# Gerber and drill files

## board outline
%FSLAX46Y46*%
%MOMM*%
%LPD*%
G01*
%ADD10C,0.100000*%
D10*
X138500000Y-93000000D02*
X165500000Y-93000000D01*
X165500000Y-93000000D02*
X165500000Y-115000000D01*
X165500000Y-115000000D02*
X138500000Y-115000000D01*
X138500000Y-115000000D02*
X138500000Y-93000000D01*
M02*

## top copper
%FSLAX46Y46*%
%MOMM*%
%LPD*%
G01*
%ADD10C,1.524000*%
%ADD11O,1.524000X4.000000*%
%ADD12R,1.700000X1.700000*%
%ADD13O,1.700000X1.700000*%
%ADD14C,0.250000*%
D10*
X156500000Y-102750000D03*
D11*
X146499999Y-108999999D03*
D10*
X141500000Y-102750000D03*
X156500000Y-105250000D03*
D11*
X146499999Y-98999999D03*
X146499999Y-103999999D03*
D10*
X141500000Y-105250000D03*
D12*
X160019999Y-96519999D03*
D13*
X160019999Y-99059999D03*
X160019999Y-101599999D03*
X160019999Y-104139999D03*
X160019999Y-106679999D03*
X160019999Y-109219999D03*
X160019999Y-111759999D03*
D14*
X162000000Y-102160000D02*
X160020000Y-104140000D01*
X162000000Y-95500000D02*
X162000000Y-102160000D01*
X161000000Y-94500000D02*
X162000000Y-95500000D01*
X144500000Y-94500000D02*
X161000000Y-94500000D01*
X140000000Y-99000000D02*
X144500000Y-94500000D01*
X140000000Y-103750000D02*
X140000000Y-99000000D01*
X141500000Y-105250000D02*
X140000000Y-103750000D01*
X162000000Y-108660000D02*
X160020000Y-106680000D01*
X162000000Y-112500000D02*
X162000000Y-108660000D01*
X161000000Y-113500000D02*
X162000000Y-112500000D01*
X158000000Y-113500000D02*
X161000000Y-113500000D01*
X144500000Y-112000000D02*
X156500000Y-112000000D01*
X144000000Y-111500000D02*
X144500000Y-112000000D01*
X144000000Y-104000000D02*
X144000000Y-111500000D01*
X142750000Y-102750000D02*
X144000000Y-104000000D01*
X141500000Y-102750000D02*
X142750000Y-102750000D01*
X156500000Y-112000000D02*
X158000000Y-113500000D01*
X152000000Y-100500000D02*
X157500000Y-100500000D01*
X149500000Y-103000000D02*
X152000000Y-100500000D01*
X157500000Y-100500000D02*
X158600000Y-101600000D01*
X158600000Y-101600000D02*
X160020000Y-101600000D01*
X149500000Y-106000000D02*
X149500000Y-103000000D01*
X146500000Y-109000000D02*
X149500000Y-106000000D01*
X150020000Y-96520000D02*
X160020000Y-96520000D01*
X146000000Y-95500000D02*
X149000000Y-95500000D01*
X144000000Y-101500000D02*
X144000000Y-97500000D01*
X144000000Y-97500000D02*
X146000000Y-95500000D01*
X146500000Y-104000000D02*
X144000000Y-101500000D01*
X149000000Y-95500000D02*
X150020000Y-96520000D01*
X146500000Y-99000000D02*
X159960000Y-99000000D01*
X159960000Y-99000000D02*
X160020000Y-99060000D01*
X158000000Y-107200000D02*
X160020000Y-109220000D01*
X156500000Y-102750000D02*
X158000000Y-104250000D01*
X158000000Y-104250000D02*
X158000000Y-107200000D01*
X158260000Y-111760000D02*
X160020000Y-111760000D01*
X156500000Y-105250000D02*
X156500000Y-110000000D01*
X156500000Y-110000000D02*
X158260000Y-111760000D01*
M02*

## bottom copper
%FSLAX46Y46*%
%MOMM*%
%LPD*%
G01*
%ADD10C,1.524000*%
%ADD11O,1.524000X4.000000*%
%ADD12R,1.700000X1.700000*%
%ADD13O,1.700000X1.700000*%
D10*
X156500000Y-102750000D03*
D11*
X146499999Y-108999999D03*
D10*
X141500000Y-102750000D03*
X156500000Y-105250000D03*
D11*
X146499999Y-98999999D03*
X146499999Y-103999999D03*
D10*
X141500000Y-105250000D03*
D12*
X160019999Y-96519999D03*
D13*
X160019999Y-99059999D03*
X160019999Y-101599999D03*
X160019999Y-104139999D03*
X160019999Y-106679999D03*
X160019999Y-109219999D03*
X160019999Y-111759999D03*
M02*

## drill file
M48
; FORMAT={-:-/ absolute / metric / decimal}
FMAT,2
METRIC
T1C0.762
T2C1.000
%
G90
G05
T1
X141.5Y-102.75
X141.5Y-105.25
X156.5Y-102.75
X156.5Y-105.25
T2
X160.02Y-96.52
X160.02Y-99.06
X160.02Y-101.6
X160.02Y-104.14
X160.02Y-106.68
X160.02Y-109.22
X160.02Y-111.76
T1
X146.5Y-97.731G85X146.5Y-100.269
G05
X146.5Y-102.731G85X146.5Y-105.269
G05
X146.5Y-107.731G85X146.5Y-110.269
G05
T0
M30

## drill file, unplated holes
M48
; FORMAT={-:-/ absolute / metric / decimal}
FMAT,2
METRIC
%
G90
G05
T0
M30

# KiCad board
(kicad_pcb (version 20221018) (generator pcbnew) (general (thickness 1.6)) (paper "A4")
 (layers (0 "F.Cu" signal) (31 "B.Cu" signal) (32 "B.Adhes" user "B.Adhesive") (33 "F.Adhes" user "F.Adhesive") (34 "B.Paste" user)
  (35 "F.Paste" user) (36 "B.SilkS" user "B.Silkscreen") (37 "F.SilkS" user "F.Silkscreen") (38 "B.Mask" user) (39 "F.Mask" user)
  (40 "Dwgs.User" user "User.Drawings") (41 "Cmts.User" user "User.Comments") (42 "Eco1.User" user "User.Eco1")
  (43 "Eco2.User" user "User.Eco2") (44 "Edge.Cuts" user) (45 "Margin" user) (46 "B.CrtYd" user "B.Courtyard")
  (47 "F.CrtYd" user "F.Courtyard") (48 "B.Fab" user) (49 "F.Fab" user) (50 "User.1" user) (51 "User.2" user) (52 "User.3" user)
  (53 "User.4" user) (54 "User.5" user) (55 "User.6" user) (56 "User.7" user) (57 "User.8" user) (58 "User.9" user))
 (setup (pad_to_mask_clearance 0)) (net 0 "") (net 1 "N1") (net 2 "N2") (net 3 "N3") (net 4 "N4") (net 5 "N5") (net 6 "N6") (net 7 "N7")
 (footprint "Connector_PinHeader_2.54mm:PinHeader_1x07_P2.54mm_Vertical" (layer "F.Cu") (at 160.02 96.52)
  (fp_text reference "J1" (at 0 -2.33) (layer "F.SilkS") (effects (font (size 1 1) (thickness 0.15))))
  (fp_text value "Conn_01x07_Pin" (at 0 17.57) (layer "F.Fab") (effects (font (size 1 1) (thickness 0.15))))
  (pad "1" thru_hole rect (at 0 0) (size 1.7 1.7) (drill 1) (layers "*.Cu" "*.Mask") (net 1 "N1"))
  (pad "2" thru_hole oval (at 0 2.54) (size 1.7 1.7) (drill 1) (layers "*.Cu" "*.Mask") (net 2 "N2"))
  (pad "3" thru_hole oval (at 0 5.08) (size 1.7 1.7) (drill 1) (layers "*.Cu" "*.Mask") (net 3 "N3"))
  (pad "4" thru_hole oval (at 0 7.62) (size 1.7 1.7) (drill 1) (layers "*.Cu" "*.Mask") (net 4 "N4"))
  (pad "5" thru_hole oval (at 0 10.16) (size 1.7 1.7) (drill 1) (layers "*.Cu" "*.Mask") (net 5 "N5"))
  (pad "6" thru_hole oval (at 0 12.7) (size 1.7 1.7) (drill 1) (layers "*.Cu" "*.Mask") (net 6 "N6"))
  (pad "7" thru_hole oval (at 0 15.24) (size 1.7 1.7) (drill 1) (layers "*.Cu" "*.Mask") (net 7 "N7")))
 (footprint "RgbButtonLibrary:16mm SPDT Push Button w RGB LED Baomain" (layer "F.Cu") (at 149 104)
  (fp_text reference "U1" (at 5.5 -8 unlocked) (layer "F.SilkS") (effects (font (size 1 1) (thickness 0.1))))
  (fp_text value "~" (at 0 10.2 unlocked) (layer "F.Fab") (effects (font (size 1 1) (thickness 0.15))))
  (pad "B" thru_hole circle (at 7.5 -1.25) (size 1.524 1.524) (drill 0.762) (layers "*.Cu" "*.Mask") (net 6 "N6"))
  (pad "COM" thru_hole oval (at -2.5 5) (size 1.524 4) (drill oval 0.762 3.3) (layers "*.Cu" "*.Mask") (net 3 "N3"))
  (pad "G" thru_hole circle (at -7.5 -1.25) (size 1.524 1.524) (drill 0.762) (layers "*.Cu" "*.Mask") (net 5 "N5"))
  (pad "GND" thru_hole circle (at 7.5 1.25) (size 1.524 1.524) (drill 0.762) (layers "*.Cu" "*.Mask") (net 7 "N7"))
  (pad "NC" thru_hole oval (at -2.5 -5) (size 1.524 4) (drill oval 0.762 3.3) (layers "*.Cu" "*.Mask") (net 2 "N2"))
  (pad "NO" thru_hole oval (at -2.5 0) (size 1.524 4) (drill oval 0.762 3.3) (layers "*.Cu" "*.Mask") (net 1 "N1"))
  (pad "R" thru_hole circle (at -7.5 1.25) (size 1.524 1.524) (drill 0.762) (layers "*.Cu" "*.Mask") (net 4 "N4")))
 (gr_rect (start 138.5 93) (end 165.5 115) (stroke (width 0.1) (type default)) (fill none) (layer "Edge.Cuts"))
 (segment (start 146.5 104) (end 144 101.5) (width 0.25) (layer "F.Cu") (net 1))
 (segment (start 150.02 96.52) (end 160.02 96.52) (width 0.25) (layer "F.Cu") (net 1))
 (segment (start 149 95.5) (end 150.02 96.52) (width 0.25) (layer "F.Cu") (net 1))
 (segment (start 144 97.5) (end 146 95.5) (width 0.25) (layer "F.Cu") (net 1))
 (segment (start 146 95.5) (end 149 95.5) (width 0.25) (layer "F.Cu") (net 1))
 (segment (start 144 101.5) (end 144 97.5) (width 0.25) (layer "F.Cu") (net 1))
 (segment (start 159.96 99) (end 160.02 99.06) (width 0.25) (layer "F.Cu") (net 2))
 (segment (start 146.5 99) (end 159.96 99) (width 0.25) (layer "F.Cu") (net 2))
 (segment (start 158.6 101.6) (end 160.02 101.6) (width 0.25) (layer "F.Cu") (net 3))
 (segment (start 149.5 103) (end 152 100.5) (width 0.25) (layer "F.Cu") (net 3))
 (segment (start 149.5 106) (end 149.5 103) (width 0.25) (layer "F.Cu") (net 3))
 (segment (start 152 100.5) (end 157.5 100.5) (width 0.25) (layer "F.Cu") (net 3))
 (segment (start 146.5 109) (end 149.5 106) (width 0.25) (layer "F.Cu") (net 3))
 (segment (start 157.5 100.5) (end 158.6 101.6) (width 0.25) (layer "F.Cu") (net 3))
 (segment (start 162 102.16) (end 160.02 104.14) (width 0.25) (layer "F.Cu") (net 4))
 (segment (start 140 99) (end 144.5 94.5) (width 0.25) (layer "F.Cu") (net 4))
 (segment (start 140 103.75) (end 140 99) (width 0.25) (layer "F.Cu") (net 4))
 (segment (start 141.5 105.25) (end 140 103.75) (width 0.25) (layer "F.Cu") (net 4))
 (segment (start 161 94.5) (end 162 95.5) (width 0.25) (layer "F.Cu") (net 4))
 (segment (start 162 95.5) (end 162 102.16) (width 0.25) (layer "F.Cu") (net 4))
 (segment (start 144.5 94.5) (end 161 94.5) (width 0.25) (layer "F.Cu") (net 4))
 (segment (start 161 113.5) (end 162 112.5) (width 0.25) (layer "F.Cu") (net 5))
 (segment (start 156.5 112) (end 158 113.5) (width 0.25) (layer "F.Cu") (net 5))
 (segment (start 162 108.66) (end 160.02 106.68) (width 0.25) (layer "F.Cu") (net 5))
 (segment (start 144 111.5) (end 144.5 112) (width 0.25) (layer "F.Cu") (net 5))
 (segment (start 144 104) (end 144 111.5) (width 0.25) (layer "F.Cu") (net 5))
 (segment (start 142.75 102.75) (end 144 104) (width 0.25) (layer "F.Cu") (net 5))
 (segment (start 141.5 102.75) (end 142.75 102.75) (width 0.25) (layer "F.Cu") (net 5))
 (segment (start 158 113.5) (end 161 113.5) (width 0.25) (layer "F.Cu") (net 5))
 (segment (start 144.5 112) (end 156.5 112) (width 0.25) (layer "F.Cu") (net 5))
 (segment (start 162 112.5) (end 162 108.66) (width 0.25) (layer "F.Cu") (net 5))
 (segment (start 158 107.2) (end 160.02 109.22) (width 0.25) (layer "F.Cu") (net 6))
 (segment (start 156.5 102.75) (end 158 104.25) (width 0.25) (layer "F.Cu") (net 6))
 (segment (start 158 104.25) (end 158 107.2) (width 0.25) (layer "F.Cu") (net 6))
 (segment (start 156.5 105.25) (end 156.5 110) (width 0.25) (layer "F.Cu") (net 7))
 (segment (start 156.5 110) (end 158.26 111.76) (width 0.25) (layer "F.Cu") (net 7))
 (segment (start 158.26 111.76) (end 160.02 111.76) (width 0.25) (layer "F.Cu") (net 7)))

